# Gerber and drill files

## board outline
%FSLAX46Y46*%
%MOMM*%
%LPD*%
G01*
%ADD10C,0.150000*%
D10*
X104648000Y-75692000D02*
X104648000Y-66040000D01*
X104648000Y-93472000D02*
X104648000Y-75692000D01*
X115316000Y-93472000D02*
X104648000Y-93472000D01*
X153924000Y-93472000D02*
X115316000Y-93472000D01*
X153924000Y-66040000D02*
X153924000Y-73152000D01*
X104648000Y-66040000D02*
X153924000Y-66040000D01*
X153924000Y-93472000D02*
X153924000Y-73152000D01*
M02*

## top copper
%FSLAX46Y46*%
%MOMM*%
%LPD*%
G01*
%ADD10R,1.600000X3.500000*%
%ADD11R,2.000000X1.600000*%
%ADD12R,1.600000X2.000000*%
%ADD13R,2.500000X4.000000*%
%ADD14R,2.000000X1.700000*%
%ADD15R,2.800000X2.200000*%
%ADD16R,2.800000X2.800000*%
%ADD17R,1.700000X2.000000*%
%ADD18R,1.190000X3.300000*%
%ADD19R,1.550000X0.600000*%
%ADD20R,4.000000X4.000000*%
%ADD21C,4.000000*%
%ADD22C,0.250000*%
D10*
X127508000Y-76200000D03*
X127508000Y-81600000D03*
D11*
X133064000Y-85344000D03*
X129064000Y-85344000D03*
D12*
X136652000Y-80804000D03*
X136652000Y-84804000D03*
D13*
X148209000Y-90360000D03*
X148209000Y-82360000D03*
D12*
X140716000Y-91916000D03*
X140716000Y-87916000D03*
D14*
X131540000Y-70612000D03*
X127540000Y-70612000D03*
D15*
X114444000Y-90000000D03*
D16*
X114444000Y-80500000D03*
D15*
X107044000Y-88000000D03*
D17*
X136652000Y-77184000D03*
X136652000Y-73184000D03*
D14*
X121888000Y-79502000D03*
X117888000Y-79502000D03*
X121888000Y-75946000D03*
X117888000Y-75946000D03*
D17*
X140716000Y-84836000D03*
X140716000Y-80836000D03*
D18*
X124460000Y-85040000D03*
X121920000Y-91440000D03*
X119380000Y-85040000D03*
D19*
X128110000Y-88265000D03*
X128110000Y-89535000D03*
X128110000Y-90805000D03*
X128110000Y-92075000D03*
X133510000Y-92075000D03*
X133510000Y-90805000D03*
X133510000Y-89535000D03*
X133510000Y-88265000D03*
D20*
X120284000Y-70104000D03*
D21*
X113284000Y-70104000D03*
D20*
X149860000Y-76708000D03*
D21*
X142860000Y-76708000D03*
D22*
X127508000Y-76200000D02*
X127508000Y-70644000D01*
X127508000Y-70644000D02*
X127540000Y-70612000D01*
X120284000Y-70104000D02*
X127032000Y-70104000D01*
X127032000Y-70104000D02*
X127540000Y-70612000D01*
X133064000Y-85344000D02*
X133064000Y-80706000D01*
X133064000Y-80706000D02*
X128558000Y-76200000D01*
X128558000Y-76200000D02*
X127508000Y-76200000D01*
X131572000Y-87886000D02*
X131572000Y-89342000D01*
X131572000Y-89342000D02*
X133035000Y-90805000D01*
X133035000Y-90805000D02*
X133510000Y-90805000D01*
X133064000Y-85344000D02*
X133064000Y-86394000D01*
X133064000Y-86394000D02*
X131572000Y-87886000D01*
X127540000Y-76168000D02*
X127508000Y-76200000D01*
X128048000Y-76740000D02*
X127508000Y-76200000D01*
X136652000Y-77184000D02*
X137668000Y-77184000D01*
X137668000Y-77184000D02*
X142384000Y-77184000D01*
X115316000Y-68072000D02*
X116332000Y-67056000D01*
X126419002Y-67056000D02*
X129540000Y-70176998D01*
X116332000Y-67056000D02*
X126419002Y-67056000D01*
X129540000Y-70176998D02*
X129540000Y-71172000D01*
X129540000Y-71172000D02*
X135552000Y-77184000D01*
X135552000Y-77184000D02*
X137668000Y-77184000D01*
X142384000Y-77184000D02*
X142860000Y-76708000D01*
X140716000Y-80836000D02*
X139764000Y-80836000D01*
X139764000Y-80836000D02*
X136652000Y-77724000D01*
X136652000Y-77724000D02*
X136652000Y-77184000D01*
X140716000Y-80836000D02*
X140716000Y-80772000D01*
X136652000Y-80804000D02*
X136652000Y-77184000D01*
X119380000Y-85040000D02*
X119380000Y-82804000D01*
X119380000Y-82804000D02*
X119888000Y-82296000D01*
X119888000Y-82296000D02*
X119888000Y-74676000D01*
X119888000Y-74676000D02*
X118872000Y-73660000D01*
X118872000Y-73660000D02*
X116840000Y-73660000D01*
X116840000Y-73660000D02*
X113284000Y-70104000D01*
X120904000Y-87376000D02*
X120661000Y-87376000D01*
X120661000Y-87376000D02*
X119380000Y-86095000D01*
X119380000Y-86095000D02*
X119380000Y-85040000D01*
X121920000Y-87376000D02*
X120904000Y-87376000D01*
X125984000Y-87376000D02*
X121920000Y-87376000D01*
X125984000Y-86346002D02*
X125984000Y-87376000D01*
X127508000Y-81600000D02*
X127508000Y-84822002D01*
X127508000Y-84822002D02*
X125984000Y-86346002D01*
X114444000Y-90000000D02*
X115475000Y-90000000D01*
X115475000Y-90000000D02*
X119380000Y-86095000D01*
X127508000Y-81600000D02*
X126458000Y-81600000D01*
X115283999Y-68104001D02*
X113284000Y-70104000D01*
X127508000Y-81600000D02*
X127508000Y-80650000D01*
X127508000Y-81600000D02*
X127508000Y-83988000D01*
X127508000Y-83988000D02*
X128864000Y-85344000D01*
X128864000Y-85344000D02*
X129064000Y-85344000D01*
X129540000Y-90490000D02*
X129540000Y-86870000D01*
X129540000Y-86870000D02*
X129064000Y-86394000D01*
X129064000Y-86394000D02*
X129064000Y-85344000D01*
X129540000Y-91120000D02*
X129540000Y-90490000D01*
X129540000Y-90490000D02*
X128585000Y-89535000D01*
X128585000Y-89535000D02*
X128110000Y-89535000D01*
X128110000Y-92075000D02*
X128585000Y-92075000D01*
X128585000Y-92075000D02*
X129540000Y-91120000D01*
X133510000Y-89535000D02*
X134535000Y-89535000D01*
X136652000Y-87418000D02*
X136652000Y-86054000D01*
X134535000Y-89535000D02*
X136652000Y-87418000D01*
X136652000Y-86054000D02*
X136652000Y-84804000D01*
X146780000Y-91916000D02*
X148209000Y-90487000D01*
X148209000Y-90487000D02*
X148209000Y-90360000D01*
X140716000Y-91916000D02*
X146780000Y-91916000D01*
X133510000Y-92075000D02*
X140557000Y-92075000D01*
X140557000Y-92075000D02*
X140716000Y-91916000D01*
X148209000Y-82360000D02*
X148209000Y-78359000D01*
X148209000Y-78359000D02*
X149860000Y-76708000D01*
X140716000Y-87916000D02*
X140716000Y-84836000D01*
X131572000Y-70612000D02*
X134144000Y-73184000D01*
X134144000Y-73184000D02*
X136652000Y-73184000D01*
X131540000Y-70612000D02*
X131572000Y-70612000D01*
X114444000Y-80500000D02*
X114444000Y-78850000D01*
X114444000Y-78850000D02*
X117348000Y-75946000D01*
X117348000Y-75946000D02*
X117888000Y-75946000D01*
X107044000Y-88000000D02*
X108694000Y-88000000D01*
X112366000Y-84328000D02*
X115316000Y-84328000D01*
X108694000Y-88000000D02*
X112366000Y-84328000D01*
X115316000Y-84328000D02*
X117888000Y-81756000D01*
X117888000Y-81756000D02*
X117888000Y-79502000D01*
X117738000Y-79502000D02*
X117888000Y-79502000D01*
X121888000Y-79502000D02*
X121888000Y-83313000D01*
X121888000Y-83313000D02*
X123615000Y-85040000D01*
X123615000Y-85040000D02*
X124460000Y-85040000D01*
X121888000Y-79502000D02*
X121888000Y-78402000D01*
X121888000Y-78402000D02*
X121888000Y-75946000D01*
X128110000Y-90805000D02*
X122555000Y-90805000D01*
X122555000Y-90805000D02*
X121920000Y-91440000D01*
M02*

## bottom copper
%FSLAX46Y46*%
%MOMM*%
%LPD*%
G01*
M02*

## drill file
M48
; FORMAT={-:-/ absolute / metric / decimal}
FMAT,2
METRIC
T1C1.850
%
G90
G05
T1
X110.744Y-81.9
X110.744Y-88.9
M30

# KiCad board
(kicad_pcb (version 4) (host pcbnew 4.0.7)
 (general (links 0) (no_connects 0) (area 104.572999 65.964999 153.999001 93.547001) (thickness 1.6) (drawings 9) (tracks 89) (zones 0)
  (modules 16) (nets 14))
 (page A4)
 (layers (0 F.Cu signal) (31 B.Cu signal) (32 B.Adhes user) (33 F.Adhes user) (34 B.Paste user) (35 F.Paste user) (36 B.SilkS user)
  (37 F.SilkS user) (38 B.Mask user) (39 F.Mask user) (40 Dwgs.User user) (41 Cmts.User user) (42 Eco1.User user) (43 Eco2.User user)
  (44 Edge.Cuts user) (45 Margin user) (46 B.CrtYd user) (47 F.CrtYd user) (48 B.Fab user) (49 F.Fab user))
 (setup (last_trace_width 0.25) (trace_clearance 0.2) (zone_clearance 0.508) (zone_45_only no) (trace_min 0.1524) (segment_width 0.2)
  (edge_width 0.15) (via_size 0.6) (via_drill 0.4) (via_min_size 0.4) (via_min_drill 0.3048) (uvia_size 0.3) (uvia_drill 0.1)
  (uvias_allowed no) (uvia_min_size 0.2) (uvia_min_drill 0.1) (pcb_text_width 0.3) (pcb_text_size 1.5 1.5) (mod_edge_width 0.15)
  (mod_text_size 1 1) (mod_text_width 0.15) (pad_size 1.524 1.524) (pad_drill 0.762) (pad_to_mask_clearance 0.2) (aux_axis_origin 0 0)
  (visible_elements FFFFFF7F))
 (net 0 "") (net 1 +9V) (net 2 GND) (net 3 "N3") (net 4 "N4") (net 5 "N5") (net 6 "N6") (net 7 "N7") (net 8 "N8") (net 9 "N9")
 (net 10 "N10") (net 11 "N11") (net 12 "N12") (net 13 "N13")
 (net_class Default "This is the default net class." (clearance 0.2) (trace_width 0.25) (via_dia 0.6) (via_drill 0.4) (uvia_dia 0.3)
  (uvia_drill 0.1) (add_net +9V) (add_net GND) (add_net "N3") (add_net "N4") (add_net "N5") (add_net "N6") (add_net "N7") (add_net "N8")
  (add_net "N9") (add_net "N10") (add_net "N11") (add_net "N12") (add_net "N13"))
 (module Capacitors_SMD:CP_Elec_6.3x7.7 (layer F.Cu) (at 127.508 78.9 270)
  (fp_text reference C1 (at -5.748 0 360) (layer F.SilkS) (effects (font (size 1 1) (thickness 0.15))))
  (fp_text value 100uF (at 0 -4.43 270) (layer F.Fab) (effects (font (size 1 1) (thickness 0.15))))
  (pad 1 smd rect (at -2.7 0 90) (size 3.5 1.6) (layers F.Cu F.Paste F.Mask) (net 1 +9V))
  (pad 2 smd rect (at 2.7 0 90) (size 3.5 1.6) (layers F.Cu F.Paste F.Mask) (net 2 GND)))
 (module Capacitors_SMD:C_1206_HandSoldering (layer F.Cu) (at 131.064 85.344 180)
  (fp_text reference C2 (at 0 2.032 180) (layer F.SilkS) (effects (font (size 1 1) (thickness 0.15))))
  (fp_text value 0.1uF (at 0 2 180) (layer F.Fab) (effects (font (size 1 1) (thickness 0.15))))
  (pad 1 smd rect (at -2 0 180) (size 2 1.6) (layers F.Cu F.Paste F.Mask) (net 1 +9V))
  (pad 2 smd rect (at 2 0 180) (size 2 1.6) (layers F.Cu F.Paste F.Mask) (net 2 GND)))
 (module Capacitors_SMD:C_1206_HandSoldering (layer F.Cu) (at 136.652 82.804 270)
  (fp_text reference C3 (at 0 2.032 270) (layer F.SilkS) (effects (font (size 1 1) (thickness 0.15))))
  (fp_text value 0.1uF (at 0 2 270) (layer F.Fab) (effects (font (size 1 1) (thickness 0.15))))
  (pad 1 smd rect (at -2 0 270) (size 2 1.6) (layers F.Cu F.Paste F.Mask) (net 2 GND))
  (pad 2 smd rect (at 2 0 270) (size 2 1.6) (layers F.Cu F.Paste F.Mask) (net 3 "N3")))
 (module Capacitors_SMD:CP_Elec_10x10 (layer F.Cu) (at 148.209 86.36 90)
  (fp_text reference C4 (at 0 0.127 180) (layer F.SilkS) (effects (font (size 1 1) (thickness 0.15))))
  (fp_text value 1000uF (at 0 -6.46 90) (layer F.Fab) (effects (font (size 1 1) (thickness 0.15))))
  (pad 1 smd rect (at -4 0 270) (size 4 2.5) (layers F.Cu F.Paste F.Mask) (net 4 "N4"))
  (pad 2 smd rect (at 4 0 270) (size 4 2.5) (layers F.Cu F.Paste F.Mask) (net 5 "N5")))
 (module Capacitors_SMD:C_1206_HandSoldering (layer F.Cu) (at 140.716 89.916 90)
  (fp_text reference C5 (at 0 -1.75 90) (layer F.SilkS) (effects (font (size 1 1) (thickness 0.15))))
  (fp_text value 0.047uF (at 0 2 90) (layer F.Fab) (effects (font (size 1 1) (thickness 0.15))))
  (pad 1 smd rect (at -2 0 90) (size 2 1.6) (layers F.Cu F.Paste F.Mask) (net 4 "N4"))
  (pad 2 smd rect (at 2 0 90) (size 2 1.6) (layers F.Cu F.Paste F.Mask) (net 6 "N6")))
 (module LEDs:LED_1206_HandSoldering (layer F.Cu) (at 129.54 70.612 180)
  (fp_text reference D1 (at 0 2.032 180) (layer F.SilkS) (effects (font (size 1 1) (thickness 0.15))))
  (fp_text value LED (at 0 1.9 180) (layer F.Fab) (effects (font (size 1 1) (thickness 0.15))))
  (pad 1 smd rect (at -2 0 180) (size 2 1.7) (layers F.Cu F.Paste F.Mask) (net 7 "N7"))
  (pad 2 smd rect (at 2 0 180) (size 2 1.7) (layers F.Cu F.Paste F.Mask) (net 1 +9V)))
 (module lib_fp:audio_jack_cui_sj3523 (layer F.Cu) (at 110.744 88.9 90)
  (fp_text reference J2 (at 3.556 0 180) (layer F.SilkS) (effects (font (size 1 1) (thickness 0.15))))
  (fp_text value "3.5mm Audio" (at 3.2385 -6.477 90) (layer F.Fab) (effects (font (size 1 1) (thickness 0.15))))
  (pad "" np_thru_hole circle (at 0 0 90) (size 1.85 1.85) (drill 1.85) (layers *.Cu *.Mask))
  (pad 1 smd rect (at -1.1 3.7 90) (size 2.2 2.8) (layers F.Cu F.Paste F.Mask) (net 2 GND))
  (pad 2 smd rect (at 8.4 3.7 90) (size 2.8 2.8) (layers F.Cu F.Paste F.Mask) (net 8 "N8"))
  (pad "" np_thru_hole circle (at 7 0 90) (size 1.85 1.85) (drill 1.85) (layers *.Cu *.Mask))
  (pad 3 smd rect (at 0.9 -3.7 90) (size 2.2 2.8) (layers F.Cu F.Paste F.Mask) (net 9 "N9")))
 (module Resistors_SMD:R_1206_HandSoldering (layer F.Cu) (at 136.652 75.184 90)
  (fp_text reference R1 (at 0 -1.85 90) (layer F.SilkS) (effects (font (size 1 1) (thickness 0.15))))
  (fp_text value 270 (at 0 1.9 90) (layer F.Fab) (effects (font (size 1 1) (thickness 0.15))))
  (pad 1 smd rect (at -2 0 90) (size 2 1.7) (layers F.Cu F.Paste F.Mask) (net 2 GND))
  (pad 2 smd rect (at 2 0 90) (size 2 1.7) (layers F.Cu F.Paste F.Mask) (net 7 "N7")))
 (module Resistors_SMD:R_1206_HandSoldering (layer F.Cu) (at 119.888 79.502 180)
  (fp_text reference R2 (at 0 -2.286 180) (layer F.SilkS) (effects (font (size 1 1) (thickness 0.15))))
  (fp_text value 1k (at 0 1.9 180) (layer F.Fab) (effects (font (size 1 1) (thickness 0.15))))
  (pad 1 smd rect (at -2 0 180) (size 2 1.7) (layers F.Cu F.Paste F.Mask) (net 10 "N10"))
  (pad 2 smd rect (at 2 0 180) (size 2 1.7) (layers F.Cu F.Paste F.Mask) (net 9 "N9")))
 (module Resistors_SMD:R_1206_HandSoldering (layer F.Cu) (at 119.888 75.946 180)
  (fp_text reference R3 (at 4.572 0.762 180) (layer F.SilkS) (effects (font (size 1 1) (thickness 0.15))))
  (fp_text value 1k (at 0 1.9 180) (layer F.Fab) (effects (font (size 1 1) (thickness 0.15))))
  (pad 1 smd rect (at -2 0 180) (size 2 1.7) (layers F.Cu F.Paste F.Mask) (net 10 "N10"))
  (pad 2 smd rect (at 2 0 180) (size 2 1.7) (layers F.Cu F.Paste F.Mask) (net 8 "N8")))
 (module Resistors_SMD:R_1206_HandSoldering (layer F.Cu) (at 140.716 82.836 90)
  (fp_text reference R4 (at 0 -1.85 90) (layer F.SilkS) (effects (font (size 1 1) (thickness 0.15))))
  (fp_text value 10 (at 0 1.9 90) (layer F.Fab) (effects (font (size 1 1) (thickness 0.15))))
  (pad 1 smd rect (at -2 0 90) (size 2 1.7) (layers F.Cu F.Paste F.Mask) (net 6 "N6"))
  (pad 2 smd rect (at 2 0 90) (size 2 1.7) (layers F.Cu F.Paste F.Mask) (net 2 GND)))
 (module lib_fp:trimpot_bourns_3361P (layer F.Cu) (at 121.92 85.04 180)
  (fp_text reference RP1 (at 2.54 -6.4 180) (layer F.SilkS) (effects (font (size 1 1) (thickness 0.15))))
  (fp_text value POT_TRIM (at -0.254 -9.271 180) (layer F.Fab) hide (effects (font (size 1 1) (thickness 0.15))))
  (pad 1 smd rect (at -2.54 0 180) (size 1.19 3.3) (layers F.Cu F.Paste F.Mask) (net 10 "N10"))
  (pad 2 smd rect (at 0 -6.4 180) (size 1.19 3.3) (layers F.Cu F.Paste F.Mask) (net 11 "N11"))
  (pad 3 smd rect (at 2.54 0 180) (size 1.19 3.3) (layers F.Cu F.Paste F.Mask) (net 2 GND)))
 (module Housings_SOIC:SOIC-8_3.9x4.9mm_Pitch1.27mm (layer F.Cu) (at 130.81 90.17)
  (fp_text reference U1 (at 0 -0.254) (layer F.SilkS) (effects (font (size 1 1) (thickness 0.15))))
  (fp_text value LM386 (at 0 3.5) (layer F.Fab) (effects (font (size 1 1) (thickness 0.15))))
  (pad 1 smd rect (at -2.7 -1.905) (size 1.55 0.6) (layers F.Cu F.Paste F.Mask) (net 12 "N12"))
  (pad 2 smd rect (at -2.7 -0.635) (size 1.55 0.6) (layers F.Cu F.Paste F.Mask) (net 2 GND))
  (pad 3 smd rect (at -2.7 0.635) (size 1.55 0.6) (layers F.Cu F.Paste F.Mask) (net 11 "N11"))
  (pad 4 smd rect (at -2.7 1.905) (size 1.55 0.6) (layers F.Cu F.Paste F.Mask) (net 2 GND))
  (pad 5 smd rect (at 2.7 1.905) (size 1.55 0.6) (layers F.Cu F.Paste F.Mask) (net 4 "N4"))
  (pad 6 smd rect (at 2.7 0.635) (size 1.55 0.6) (layers F.Cu F.Paste F.Mask) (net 1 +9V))
  (pad 7 smd rect (at 2.7 -0.635) (size 1.55 0.6) (layers F.Cu F.Paste F.Mask) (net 3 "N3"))
  (pad 8 smd rect (at 2.7 -1.905) (size 1.55 0.6) (layers F.Cu F.Paste F.Mask) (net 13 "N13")))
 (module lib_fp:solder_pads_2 (layer F.Cu) (at 120.284 70.104 180)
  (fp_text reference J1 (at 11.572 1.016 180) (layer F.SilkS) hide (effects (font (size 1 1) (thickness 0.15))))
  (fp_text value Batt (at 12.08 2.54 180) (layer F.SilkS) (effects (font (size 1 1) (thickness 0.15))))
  (pad 1 smd rect (at 0 0 180) (size 4 4) (layers F.Cu F.Paste F.Mask) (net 1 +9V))
  (pad 2 smd circle (at 7 0 180) (size 4 4) (layers F.Cu F.Paste F.Mask) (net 2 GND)))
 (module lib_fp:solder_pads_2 (layer F.Cu) (at 149.86 76.708 180)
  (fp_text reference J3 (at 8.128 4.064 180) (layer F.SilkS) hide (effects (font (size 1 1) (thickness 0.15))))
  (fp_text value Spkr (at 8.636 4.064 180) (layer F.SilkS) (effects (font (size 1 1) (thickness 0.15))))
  (pad 1 smd rect (at 0 0 180) (size 4 4) (layers F.Cu F.Paste F.Mask) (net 5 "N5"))
  (pad 2 smd circle (at 7 0 180) (size 4 4) (layers F.Cu F.Paste F.Mask) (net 2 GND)))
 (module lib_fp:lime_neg (layer F.Cu) (at 148.336 69.088)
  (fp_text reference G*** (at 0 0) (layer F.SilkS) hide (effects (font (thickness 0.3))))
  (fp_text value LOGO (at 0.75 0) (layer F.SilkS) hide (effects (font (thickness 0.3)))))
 (gr_line (start 104.648 75.692) (end 104.648 66.04) (layer Edge.Cuts) (width 0.15))
 (gr_line (start 104.648 93.472) (end 104.648 75.692) (layer Edge.Cuts) (width 0.15))
 (gr_line (start 115.316 93.472) (end 104.648 93.472) (layer Edge.Cuts) (width 0.15))
 (gr_line (start 153.924 93.472) (end 115.316 93.472) (layer Edge.Cuts) (width 0.15))
 (gr_line (start 153.924 66.04) (end 153.924 73.152) (layer Edge.Cuts) (width 0.15))
 (gr_line (start 104.648 66.04) (end 153.924 66.04) (layer Edge.Cuts) (width 0.15))
 (gr_line (start 153.924 93.472) (end 153.924 73.152) (layer Edge.Cuts) (width 0.15))
 (segment (start 127.508 76.2) (end 127.508 70.644) (width 0.25) (layer F.Cu) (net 1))
 (segment (start 127.508 70.644) (end 127.54 70.612) (width 0.25) (layer F.Cu) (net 1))
 (segment (start 120.284 70.104) (end 127.032 70.104) (width 0.25) (layer F.Cu) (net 1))
 (segment (start 127.032 70.104) (end 127.54 70.612) (width 0.25) (layer F.Cu) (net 1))
 (segment (start 133.064 85.344) (end 133.064 80.706) (width 0.25) (layer F.Cu) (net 1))
 (segment (start 133.064 80.706) (end 128.558 76.2) (width 0.25) (layer F.Cu) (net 1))
 (segment (start 128.558 76.2) (end 127.508 76.2) (width 0.25) (layer F.Cu) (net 1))
 (segment (start 131.572 87.886) (end 131.572 89.342) (width 0.25) (layer F.Cu) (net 1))
 (segment (start 131.572 89.342) (end 133.035 90.805) (width 0.25) (layer F.Cu) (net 1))
 (segment (start 133.035 90.805) (end 133.51 90.805) (width 0.25) (layer F.Cu) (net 1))
 (segment (start 133.064 85.344) (end 133.064 86.394) (width 0.25) (layer F.Cu) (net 1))
 (segment (start 133.064 86.394) (end 131.572 87.886) (width 0.25) (layer F.Cu) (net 1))
 (segment (start 127.54 76.168) (end 127.508 76.2) (width 0.25) (layer F.Cu) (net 1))
 (segment (start 128.048 76.74) (end 127.508 76.2) (width 0.25) (layer F.Cu) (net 1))
 (segment (start 136.652 77.184) (end 137.668 77.184) (width 0.25) (layer F.Cu) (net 2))
 (segment (start 137.668 77.184) (end 142.384 77.184) (width 0.25) (layer F.Cu) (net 2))
 (segment (start 115.316 68.072) (end 116.332 67.056) (width 0.25) (layer F.Cu) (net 2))
 (segment (start 126.419002 67.056) (end 129.54 70.176998) (width 0.25) (layer F.Cu) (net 2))
 (segment (start 116.332 67.056) (end 126.419002 67.056) (width 0.25) (layer F.Cu) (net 2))
 (segment (start 129.54 70.176998) (end 129.54 71.172) (width 0.25) (layer F.Cu) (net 2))
 (segment (start 129.54 71.172) (end 135.552 77.184) (width 0.25) (layer F.Cu) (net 2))
 (segment (start 135.552 77.184) (end 137.668 77.184) (width 0.25) (layer F.Cu) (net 2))
 (segment (start 142.384 77.184) (end 142.86 76.708) (width 0.25) (layer F.Cu) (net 2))
 (segment (start 140.716 80.836) (end 139.764 80.836) (width 0.25) (layer F.Cu) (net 2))
 (segment (start 139.764 80.836) (end 136.652 77.724) (width 0.25) (layer F.Cu) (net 2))
 (segment (start 136.652 77.724) (end 136.652 77.184) (width 0.25) (layer F.Cu) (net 2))
 (segment (start 140.716 80.836) (end 140.716 80.772) (width 0.25) (layer F.Cu) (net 2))
 (segment (start 136.652 80.804) (end 136.652 77.184) (width 0.25) (layer F.Cu) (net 2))
 (segment (start 119.38 85.04) (end 119.38 82.804) (width 0.25) (layer F.Cu) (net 2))
 (segment (start 119.38 82.804) (end 119.888 82.296) (width 0.25) (layer F.Cu) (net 2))
 (segment (start 119.888 82.296) (end 119.888 74.676) (width 0.25) (layer F.Cu) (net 2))
 (segment (start 119.888 74.676) (end 118.872 73.66) (width 0.25) (layer F.Cu) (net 2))
 (segment (start 118.872 73.66) (end 116.84 73.66) (width 0.25) (layer F.Cu) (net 2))
 (segment (start 116.84 73.66) (end 113.284 70.104) (width 0.25) (layer F.Cu) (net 2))
 (segment (start 120.904 87.376) (end 120.661 87.376) (width 0.25) (layer F.Cu) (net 2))
 (segment (start 120.661 87.376) (end 119.38 86.095) (width 0.25) (layer F.Cu) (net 2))
 (segment (start 119.38 86.095) (end 119.38 85.04) (width 0.25) (layer F.Cu) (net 2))
 (segment (start 121.92 87.376) (end 120.904 87.376) (width 0.25) (layer F.Cu) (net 2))
 (segment (start 125.984 87.376) (end 121.92 87.376) (width 0.25) (layer F.Cu) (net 2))
 (segment (start 125.984 86.346002) (end 125.984 87.376) (width 0.25) (layer F.Cu) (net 2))
 (segment (start 127.508 81.6) (end 127.508 84.822002) (width 0.25) (layer F.Cu) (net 2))
 (segment (start 127.508 84.822002) (end 125.984 86.346002) (width 0.25) (layer F.Cu) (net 2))
 (segment (start 114.444 90) (end 115.475 90) (width 0.25) (layer F.Cu) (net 2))
 (segment (start 115.475 90) (end 119.38 86.095) (width 0.25) (layer F.Cu) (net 2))
 (segment (start 127.508 81.6) (end 126.458 81.6) (width 0.25) (layer F.Cu) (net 2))
 (segment (start 115.283999 68.104001) (end 113.284 70.104) (width 0.25) (layer F.Cu) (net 2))
 (segment (start 127.508 81.6) (end 127.508 80.65) (width 0.25) (layer F.Cu) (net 2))
 (segment (start 127.508 81.6) (end 127.508 83.988) (width 0.25) (layer F.Cu) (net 2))
 (segment (start 127.508 83.988) (end 128.864 85.344) (width 0.25) (layer F.Cu) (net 2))
 (segment (start 128.864 85.344) (end 129.064 85.344) (width 0.25) (layer F.Cu) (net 2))
 (segment (start 129.54 90.49) (end 129.54 86.87) (width 0.25) (layer F.Cu) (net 2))
 (segment (start 129.54 86.87) (end 129.064 86.394) (width 0.25) (layer F.Cu) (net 2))
 (segment (start 129.064 86.394) (end 129.064 85.344) (width 0.25) (layer F.Cu) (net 2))
 (segment (start 129.54 91.12) (end 129.54 90.49) (width 0.25) (layer F.Cu) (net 2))
 (segment (start 129.54 90.49) (end 128.585 89.535) (width 0.25) (layer F.Cu) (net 2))
 (segment (start 128.585 89.535) (end 128.11 89.535) (width 0.25) (layer F.Cu) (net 2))
 (segment (start 128.11 92.075) (end 128.585 92.075) (width 0.25) (layer F.Cu) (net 2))
 (segment (start 128.585 92.075) (end 129.54 91.12) (width 0.25) (layer F.Cu) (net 2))
 (segment (start 133.51 89.535) (end 134.535 89.535) (width 0.25) (layer F.Cu) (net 3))
 (segment (start 136.652 87.418) (end 136.652 86.054) (width 0.25) (layer F.Cu) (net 3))
 (segment (start 134.535 89.535) (end 136.652 87.418) (width 0.25) (layer F.Cu) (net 3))
 (segment (start 136.652 86.054) (end 136.652 84.804) (width 0.25) (layer F.Cu) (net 3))
 (segment (start 146.78 91.916) (end 148.209 90.487) (width 0.25) (layer F.Cu) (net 4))
 (segment (start 148.209 90.487) (end 148.209 90.36) (width 0.25) (layer F.Cu) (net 4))
 (segment (start 140.716 91.916) (end 146.78 91.916) (width 0.25) (layer F.Cu) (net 4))
 (segment (start 133.51 92.075) (end 140.557 92.075) (width 0.25) (layer F.Cu) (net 4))
 (segment (start 140.557 92.075) (end 140.716 91.916) (width 0.25) (layer F.Cu) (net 4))
 (segment (start 148.209 82.36) (end 148.209 78.359) (width 0.25) (layer F.Cu) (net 5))
 (segment (start 148.209 78.359) (end 149.86 76.708) (width 0.25) (layer F.Cu) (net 5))
 (segment (start 140.716 87.916) (end 140.716 84.836) (width 0.25) (layer F.Cu) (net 6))
 (segment (start 131.572 70.612) (end 134.144 73.184) (width 0.25) (layer F.Cu) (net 7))
 (segment (start 134.144 73.184) (end 136.652 73.184) (width 0.25) (layer F.Cu) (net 7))
 (segment (start 131.54 70.612) (end 131.572 70.612) (width 0.25) (layer F.Cu) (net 7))
 (segment (start 114.444 80.5) (end 114.444 78.85) (width 0.25) (layer F.Cu) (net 8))
 (segment (start 114.444 78.85) (end 117.348 75.946) (width 0.25) (layer F.Cu) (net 8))
 (segment (start 117.348 75.946) (end 117.888 75.946) (width 0.25) (layer F.Cu) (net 8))
 (segment (start 107.044 88) (end 108.694 88) (width 0.25) (layer F.Cu) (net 9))
 (segment (start 112.366 84.328) (end 115.316 84.328) (width 0.25) (layer F.Cu) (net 9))
 (segment (start 108.694 88) (end 112.366 84.328) (width 0.25) (layer F.Cu) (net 9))
 (segment (start 115.316 84.328) (end 117.888 81.756) (width 0.25) (layer F.Cu) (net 9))
 (segment (start 117.888 81.756) (end 117.888 79.502) (width 0.25) (layer F.Cu) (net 9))
 (segment (start 117.738 79.502) (end 117.888 79.502) (width 0.25) (layer F.Cu) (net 9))
 (segment (start 121.888 79.502) (end 121.888 83.313) (width 0.25) (layer F.Cu) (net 10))
 (segment (start 121.888 83.313) (end 123.615 85.04) (width 0.25) (layer F.Cu) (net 10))
 (segment (start 123.615 85.04) (end 124.46 85.04) (width 0.25) (layer F.Cu) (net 10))
 (segment (start 121.888 79.502) (end 121.888 78.402) (width 0.25) (layer F.Cu) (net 10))
 (segment (start 121.888 78.402) (end 121.888 75.946) (width 0.25) (layer F.Cu) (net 10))
 (segment (start 128.11 90.805) (end 122.555 90.805) (width 0.25) (layer F.Cu) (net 11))
 (segment (start 122.555 90.805) (end 121.92 91.44) (width 0.25) (layer F.Cu) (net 11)))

